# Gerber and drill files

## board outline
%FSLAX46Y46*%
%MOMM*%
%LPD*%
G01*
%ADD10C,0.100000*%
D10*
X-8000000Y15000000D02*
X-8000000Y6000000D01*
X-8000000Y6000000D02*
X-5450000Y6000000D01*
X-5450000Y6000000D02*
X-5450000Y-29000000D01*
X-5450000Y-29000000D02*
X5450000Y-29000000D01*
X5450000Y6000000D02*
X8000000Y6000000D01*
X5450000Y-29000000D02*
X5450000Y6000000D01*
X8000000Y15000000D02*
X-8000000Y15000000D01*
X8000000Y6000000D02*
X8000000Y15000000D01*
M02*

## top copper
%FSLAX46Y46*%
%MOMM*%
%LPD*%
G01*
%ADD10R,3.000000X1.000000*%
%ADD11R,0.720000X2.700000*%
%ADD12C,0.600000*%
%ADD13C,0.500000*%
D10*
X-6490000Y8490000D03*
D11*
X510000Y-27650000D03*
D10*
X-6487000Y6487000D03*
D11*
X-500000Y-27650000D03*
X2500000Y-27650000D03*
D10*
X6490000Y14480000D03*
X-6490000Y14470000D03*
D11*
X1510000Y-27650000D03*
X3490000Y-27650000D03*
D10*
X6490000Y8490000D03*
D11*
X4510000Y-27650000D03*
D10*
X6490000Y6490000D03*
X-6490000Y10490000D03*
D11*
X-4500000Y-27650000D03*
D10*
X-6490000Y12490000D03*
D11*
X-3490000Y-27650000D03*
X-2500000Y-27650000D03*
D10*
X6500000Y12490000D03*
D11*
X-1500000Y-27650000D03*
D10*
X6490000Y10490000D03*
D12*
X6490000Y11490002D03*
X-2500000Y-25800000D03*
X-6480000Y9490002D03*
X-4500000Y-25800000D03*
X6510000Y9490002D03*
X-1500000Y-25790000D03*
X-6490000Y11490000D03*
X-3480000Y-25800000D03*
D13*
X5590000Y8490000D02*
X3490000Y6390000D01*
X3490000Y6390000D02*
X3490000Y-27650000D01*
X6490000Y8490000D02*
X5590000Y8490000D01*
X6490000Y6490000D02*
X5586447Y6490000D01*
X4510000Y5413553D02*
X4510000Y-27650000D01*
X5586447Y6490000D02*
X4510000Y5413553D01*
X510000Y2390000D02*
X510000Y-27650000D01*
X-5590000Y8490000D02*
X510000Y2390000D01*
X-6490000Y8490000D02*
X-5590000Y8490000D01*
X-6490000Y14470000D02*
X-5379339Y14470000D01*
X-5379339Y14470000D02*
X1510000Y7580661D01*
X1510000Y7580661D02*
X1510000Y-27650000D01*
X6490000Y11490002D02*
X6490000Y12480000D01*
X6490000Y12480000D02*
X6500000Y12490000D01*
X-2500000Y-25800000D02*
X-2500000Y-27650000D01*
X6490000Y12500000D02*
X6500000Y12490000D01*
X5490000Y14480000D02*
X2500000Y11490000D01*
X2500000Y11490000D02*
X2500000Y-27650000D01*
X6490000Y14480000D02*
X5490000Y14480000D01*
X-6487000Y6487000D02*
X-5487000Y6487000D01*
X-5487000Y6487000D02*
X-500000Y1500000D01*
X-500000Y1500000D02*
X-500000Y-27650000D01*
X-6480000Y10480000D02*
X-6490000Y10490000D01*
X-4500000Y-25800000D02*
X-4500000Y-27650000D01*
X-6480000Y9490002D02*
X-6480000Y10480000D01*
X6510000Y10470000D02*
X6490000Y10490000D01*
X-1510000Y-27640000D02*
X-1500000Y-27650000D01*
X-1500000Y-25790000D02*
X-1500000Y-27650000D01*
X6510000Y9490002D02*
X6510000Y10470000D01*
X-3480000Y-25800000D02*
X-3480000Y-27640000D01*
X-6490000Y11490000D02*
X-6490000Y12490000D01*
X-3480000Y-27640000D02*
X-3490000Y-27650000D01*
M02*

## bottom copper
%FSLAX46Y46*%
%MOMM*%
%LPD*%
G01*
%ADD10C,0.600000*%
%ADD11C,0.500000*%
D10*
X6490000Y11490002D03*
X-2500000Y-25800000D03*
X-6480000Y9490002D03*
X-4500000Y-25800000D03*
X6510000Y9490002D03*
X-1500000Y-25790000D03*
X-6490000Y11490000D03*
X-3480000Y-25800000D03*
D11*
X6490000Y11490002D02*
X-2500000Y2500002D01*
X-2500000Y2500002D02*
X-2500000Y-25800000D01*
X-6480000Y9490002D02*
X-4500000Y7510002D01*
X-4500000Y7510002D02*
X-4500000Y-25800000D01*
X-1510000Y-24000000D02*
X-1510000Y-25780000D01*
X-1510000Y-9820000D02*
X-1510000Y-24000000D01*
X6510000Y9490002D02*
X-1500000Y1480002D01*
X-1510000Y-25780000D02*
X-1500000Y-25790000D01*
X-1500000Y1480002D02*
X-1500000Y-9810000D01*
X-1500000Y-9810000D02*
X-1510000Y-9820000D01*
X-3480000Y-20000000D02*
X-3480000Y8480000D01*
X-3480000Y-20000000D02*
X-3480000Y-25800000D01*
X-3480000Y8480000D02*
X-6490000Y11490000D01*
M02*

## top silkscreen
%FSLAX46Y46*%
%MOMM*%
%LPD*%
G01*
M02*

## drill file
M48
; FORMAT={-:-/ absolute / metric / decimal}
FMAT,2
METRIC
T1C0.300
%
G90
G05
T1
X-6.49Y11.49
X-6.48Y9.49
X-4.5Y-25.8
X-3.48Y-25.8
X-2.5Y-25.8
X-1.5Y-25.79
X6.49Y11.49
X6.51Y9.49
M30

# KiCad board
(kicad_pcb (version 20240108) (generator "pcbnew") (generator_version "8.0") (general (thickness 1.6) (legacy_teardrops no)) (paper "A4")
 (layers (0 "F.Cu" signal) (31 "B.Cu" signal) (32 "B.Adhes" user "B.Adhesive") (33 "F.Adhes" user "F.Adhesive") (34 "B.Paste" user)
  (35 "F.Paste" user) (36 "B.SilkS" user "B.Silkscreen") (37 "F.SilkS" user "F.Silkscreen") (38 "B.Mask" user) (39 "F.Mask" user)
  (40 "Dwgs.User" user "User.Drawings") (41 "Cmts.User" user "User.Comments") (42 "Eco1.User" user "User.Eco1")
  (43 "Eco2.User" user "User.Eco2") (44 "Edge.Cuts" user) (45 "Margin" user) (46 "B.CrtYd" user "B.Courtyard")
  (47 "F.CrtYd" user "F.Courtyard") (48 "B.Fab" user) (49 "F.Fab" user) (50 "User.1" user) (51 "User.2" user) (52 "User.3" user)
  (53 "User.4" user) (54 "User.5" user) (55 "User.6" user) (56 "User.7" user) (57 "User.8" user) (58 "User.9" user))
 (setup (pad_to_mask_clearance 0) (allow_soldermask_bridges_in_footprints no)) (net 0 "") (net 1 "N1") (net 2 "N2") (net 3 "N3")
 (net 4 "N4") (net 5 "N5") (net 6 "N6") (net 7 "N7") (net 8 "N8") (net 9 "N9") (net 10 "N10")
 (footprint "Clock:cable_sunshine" (layer "F.Cu") (at 0 0)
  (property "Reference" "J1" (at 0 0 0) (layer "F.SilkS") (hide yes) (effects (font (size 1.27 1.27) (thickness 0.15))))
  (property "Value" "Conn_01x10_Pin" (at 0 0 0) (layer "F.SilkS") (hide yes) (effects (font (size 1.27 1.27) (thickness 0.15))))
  (fp_line (start -8 -15) (end -8 -6) (stroke (width 0.1) (type solid)) (layer "Edge.Cuts"))
  (fp_line (start -8 -6) (end -5.45 -6) (stroke (width 0.1) (type solid)) (layer "Edge.Cuts"))
  (fp_line (start -5.45 -6) (end -5.45 29) (stroke (width 0.1) (type solid)) (layer "Edge.Cuts"))
  (fp_line (start -5.45 29) (end 5.45 29) (stroke (width 0.1) (type solid)) (layer "Edge.Cuts"))
  (fp_line (start 5.45 -6) (end 8 -6) (stroke (width 0.1) (type solid)) (layer "Edge.Cuts"))
  (fp_line (start 5.45 29) (end 5.45 -6) (stroke (width 0.1) (type solid)) (layer "Edge.Cuts"))
  (fp_line (start 8 -15) (end -8 -15) (stroke (width 0.1) (type solid)) (layer "Edge.Cuts"))
  (fp_line (start 8 -6) (end 8 -15) (stroke (width 0.1) (type solid)) (layer "Edge.Cuts"))
  (pad "G1B" smd rect (at -6.49 -8.49) (size 3 1) (layers "F.Cu" "F.Paste" "F.Mask") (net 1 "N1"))
  (pad "G1B" smd rect (at 0.51 27.65) (size 0.72 2.7) (layers "F.Cu" "F.Paste" "F.Mask") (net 1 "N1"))
  (pad "G1T" smd rect (at -6.487 -6.487) (size 3 1) (layers "F.Cu" "F.Paste" "F.Mask") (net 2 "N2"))
  (pad "G1T" smd rect (at -0.5 27.65) (size 0.72 2.7) (layers "F.Cu" "F.Paste" "F.Mask") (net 2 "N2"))
  (pad "G2B" smd rect (at 2.5 27.65) (size 0.72 2.7) (layers "F.Cu" "F.Paste" "F.Mask") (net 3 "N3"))
  (pad "G2B" smd rect (at 6.49 -14.48) (size 3 1) (layers "F.Cu" "F.Paste" "F.Mask") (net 3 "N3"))
  (pad "G2T" smd rect (at -6.49 -14.47) (size 3 1) (layers "F.Cu" "F.Paste" "F.Mask") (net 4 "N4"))
  (pad "G2T" smd rect (at 1.51 27.65) (size 0.72 2.7) (layers "F.Cu" "F.Paste" "F.Mask") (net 4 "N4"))
  (pad "G3B" smd rect (at 3.49 27.65) (size 0.72 2.7) (layers "F.Cu" "F.Paste" "F.Mask") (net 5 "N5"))
  (pad "G3B" smd rect (at 6.49 -8.49) (size 3 1) (layers "F.Cu" "F.Paste" "F.Mask") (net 5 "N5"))
  (pad "G3T" smd rect (at 4.51 27.65) (size 0.72 2.7) (layers "F.Cu" "F.Paste" "F.Mask") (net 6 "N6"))
  (pad "G3T" smd rect (at 6.49 -6.49) (size 3 1) (layers "F.Cu" "F.Paste" "F.Mask") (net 6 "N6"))
  (pad "H1" smd rect (at -6.49 -10.49) (size 3 1) (layers "F.Cu" "F.Paste" "F.Mask") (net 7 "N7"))
  (pad "H1" smd rect (at -4.5 27.65) (size 0.72 2.7) (layers "F.Cu" "F.Paste" "F.Mask") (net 7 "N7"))
  (pad "H2" smd rect (at -6.49 -12.49) (size 3 1) (layers "F.Cu" "F.Paste" "F.Mask") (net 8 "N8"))
  (pad "H2" smd rect (at -3.49 27.65) (size 0.72 2.7) (layers "F.Cu" "F.Paste" "F.Mask") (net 8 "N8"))
  (pad "H3" smd rect (at -2.5 27.65) (size 0.72 2.7) (layers "F.Cu" "F.Paste" "F.Mask") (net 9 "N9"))
  (pad "H3" smd rect (at 6.5 -12.49) (size 3 1) (layers "F.Cu" "F.Paste" "F.Mask") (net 9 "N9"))
  (pad "H4" smd rect (at -1.5 27.65) (size 0.72 2.7) (layers "F.Cu" "F.Paste" "F.Mask") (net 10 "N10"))
  (pad "H4" smd rect (at 6.49 -10.49) (size 3 1) (layers "F.Cu" "F.Paste" "F.Mask") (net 10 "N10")))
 (segment (start 5.59 -8.49) (end 3.49 -6.39) (width 0.5) (layer "F.Cu") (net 5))
 (segment (start 3.49 -6.39) (end 3.49 27.65) (width 0.5) (layer "F.Cu") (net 5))
 (segment (start 6.49 -8.49) (end 5.59 -8.49) (width 0.5) (layer "F.Cu") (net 5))
 (segment (start 6.49 -6.49) (end 5.586447 -6.49) (width 0.5) (layer "F.Cu") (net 6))
 (segment (start 4.51 -5.413553) (end 4.51 27.65) (width 0.5) (layer "F.Cu") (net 6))
 (segment (start 5.586447 -6.49) (end 4.51 -5.413553) (width 0.5) (layer "F.Cu") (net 6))
 (segment (start 0.51 -2.39) (end 0.51 27.65) (width 0.5) (layer "F.Cu") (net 1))
 (segment (start -5.59 -8.49) (end 0.51 -2.39) (width 0.5) (layer "F.Cu") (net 1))
 (segment (start -6.49 -8.49) (end -5.59 -8.49) (width 0.5) (layer "F.Cu") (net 1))
 (segment (start -6.49 -14.47) (end -5.379339 -14.47) (width 0.5) (layer "F.Cu") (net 4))
 (segment (start -5.379339 -14.47) (end 1.51 -7.580661) (width 0.5) (layer "F.Cu") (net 4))
 (segment (start 1.51 -7.580661) (end 1.51 27.65) (width 0.5) (layer "F.Cu") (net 4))
 (segment (start 6.49 -11.490002) (end 6.49 -12.48) (width 0.5) (layer "F.Cu") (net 9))
 (segment (start 6.49 -12.48) (end 6.5 -12.49) (width 0.5) (layer "F.Cu") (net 9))
 (segment (start -2.5 25.8) (end -2.5 27.65) (width 0.5) (layer "F.Cu") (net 9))
 (segment (start 6.49 -12.5) (end 6.5 -12.49) (width 0.5) (layer "F.Cu") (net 9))
 (via (at 6.49 -11.490002) (size 0.6) (drill 0.3) (layers "F.Cu" "B.Cu") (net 9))
 (via (at -2.5 25.8) (size 0.6) (drill 0.3) (layers "F.Cu" "B.Cu") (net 9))
 (segment (start 6.49 -11.490002) (end -2.5 -2.500002) (width 0.5) (layer "B.Cu") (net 9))
 (segment (start -2.5 -2.500002) (end -2.5 25.8) (width 0.5) (layer "B.Cu") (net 9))
 (segment (start 5.49 -14.48) (end 2.5 -11.49) (width 0.5) (layer "F.Cu") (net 3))
 (segment (start 2.5 -11.49) (end 2.5 27.65) (width 0.5) (layer "F.Cu") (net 3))
 (segment (start 6.49 -14.48) (end 5.49 -14.48) (width 0.5) (layer "F.Cu") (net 3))
 (segment (start -6.487 -6.487) (end -5.487 -6.487) (width 0.5) (layer "F.Cu") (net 2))
 (segment (start -5.487 -6.487) (end -0.5 -1.5) (width 0.5) (layer "F.Cu") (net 2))
 (segment (start -0.5 -1.5) (end -0.5 27.65) (width 0.5) (layer "F.Cu") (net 2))
 (segment (start -6.48 -10.48) (end -6.49 -10.49) (width 0.5) (layer "F.Cu") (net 7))
 (segment (start -4.5 25.8) (end -4.5 27.65) (width 0.5) (layer "F.Cu") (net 7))
 (segment (start -6.48 -9.490002) (end -6.48 -10.48) (width 0.5) (layer "F.Cu") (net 7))
 (via (at -6.48 -9.490002) (size 0.6) (drill 0.3) (layers "F.Cu" "B.Cu") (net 7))
 (via (at -4.5 25.8) (size 0.6) (drill 0.3) (layers "F.Cu" "B.Cu") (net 7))
 (segment (start -6.48 -9.490002) (end -4.5 -7.510002) (width 0.5) (layer "B.Cu") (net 7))
 (segment (start -4.5 -7.510002) (end -4.5 25.8) (width 0.5) (layer "B.Cu") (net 7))
 (segment (start 6.51 -10.47) (end 6.49 -10.49) (width 0.5) (layer "F.Cu") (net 10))
 (segment (start -1.51 27.64) (end -1.5 27.65) (width 0.5) (layer "F.Cu") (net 10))
 (segment (start -1.5 25.79) (end -1.5 27.65) (width 0.5) (layer "F.Cu") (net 10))
 (segment (start 6.51 -9.490002) (end 6.51 -10.47) (width 0.5) (layer "F.Cu") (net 10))
 (via (at 6.51 -9.490002) (size 0.6) (drill 0.3) (layers "F.Cu" "B.Cu") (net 10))
 (via (at -1.5 25.79) (size 0.6) (drill 0.3) (layers "F.Cu" "B.Cu") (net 10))
 (segment (start -1.51 24) (end -1.51 25.78) (width 0.5) (layer "B.Cu") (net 10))
 (segment (start -1.51 9.82) (end -1.51 24) (width 0.5) (layer "B.Cu") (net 10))
 (segment (start 6.51 -9.490002) (end -1.5 -1.480002) (width 0.5) (layer "B.Cu") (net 10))
 (segment (start -1.51 25.78) (end -1.5 25.79) (width 0.5) (layer "B.Cu") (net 10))
 (segment (start -1.5 -1.480002) (end -1.5 9.81) (width 0.5) (layer "B.Cu") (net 10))
 (segment (start -1.5 9.81) (end -1.51 9.82) (width 0.5) (layer "B.Cu") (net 10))
 (segment (start -3.48 25.8) (end -3.48 27.64) (width 0.5) (layer "F.Cu") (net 8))
 (segment (start -6.49 -11.49) (end -6.49 -12.49) (width 0.5) (layer "F.Cu") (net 8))
 (segment (start -3.48 27.64) (end -3.49 27.65) (width 0.5) (layer "F.Cu") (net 8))
 (via (at -6.49 -11.49) (size 0.6) (drill 0.3) (layers "F.Cu" "B.Cu") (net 8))
 (via (at -3.48 25.8) (size 0.6) (drill 0.3) (layers "F.Cu" "B.Cu") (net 8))
 (segment (start -3.48 20) (end -3.48 -8.48) (width 0.5) (layer "B.Cu") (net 8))
 (segment (start -3.48 20) (end -3.48 25.8) (width 0.5) (layer "B.Cu") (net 8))
 (segment (start -3.48 -8.48) (end -6.49 -11.49) (width 0.5) (layer "B.Cu") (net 8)))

